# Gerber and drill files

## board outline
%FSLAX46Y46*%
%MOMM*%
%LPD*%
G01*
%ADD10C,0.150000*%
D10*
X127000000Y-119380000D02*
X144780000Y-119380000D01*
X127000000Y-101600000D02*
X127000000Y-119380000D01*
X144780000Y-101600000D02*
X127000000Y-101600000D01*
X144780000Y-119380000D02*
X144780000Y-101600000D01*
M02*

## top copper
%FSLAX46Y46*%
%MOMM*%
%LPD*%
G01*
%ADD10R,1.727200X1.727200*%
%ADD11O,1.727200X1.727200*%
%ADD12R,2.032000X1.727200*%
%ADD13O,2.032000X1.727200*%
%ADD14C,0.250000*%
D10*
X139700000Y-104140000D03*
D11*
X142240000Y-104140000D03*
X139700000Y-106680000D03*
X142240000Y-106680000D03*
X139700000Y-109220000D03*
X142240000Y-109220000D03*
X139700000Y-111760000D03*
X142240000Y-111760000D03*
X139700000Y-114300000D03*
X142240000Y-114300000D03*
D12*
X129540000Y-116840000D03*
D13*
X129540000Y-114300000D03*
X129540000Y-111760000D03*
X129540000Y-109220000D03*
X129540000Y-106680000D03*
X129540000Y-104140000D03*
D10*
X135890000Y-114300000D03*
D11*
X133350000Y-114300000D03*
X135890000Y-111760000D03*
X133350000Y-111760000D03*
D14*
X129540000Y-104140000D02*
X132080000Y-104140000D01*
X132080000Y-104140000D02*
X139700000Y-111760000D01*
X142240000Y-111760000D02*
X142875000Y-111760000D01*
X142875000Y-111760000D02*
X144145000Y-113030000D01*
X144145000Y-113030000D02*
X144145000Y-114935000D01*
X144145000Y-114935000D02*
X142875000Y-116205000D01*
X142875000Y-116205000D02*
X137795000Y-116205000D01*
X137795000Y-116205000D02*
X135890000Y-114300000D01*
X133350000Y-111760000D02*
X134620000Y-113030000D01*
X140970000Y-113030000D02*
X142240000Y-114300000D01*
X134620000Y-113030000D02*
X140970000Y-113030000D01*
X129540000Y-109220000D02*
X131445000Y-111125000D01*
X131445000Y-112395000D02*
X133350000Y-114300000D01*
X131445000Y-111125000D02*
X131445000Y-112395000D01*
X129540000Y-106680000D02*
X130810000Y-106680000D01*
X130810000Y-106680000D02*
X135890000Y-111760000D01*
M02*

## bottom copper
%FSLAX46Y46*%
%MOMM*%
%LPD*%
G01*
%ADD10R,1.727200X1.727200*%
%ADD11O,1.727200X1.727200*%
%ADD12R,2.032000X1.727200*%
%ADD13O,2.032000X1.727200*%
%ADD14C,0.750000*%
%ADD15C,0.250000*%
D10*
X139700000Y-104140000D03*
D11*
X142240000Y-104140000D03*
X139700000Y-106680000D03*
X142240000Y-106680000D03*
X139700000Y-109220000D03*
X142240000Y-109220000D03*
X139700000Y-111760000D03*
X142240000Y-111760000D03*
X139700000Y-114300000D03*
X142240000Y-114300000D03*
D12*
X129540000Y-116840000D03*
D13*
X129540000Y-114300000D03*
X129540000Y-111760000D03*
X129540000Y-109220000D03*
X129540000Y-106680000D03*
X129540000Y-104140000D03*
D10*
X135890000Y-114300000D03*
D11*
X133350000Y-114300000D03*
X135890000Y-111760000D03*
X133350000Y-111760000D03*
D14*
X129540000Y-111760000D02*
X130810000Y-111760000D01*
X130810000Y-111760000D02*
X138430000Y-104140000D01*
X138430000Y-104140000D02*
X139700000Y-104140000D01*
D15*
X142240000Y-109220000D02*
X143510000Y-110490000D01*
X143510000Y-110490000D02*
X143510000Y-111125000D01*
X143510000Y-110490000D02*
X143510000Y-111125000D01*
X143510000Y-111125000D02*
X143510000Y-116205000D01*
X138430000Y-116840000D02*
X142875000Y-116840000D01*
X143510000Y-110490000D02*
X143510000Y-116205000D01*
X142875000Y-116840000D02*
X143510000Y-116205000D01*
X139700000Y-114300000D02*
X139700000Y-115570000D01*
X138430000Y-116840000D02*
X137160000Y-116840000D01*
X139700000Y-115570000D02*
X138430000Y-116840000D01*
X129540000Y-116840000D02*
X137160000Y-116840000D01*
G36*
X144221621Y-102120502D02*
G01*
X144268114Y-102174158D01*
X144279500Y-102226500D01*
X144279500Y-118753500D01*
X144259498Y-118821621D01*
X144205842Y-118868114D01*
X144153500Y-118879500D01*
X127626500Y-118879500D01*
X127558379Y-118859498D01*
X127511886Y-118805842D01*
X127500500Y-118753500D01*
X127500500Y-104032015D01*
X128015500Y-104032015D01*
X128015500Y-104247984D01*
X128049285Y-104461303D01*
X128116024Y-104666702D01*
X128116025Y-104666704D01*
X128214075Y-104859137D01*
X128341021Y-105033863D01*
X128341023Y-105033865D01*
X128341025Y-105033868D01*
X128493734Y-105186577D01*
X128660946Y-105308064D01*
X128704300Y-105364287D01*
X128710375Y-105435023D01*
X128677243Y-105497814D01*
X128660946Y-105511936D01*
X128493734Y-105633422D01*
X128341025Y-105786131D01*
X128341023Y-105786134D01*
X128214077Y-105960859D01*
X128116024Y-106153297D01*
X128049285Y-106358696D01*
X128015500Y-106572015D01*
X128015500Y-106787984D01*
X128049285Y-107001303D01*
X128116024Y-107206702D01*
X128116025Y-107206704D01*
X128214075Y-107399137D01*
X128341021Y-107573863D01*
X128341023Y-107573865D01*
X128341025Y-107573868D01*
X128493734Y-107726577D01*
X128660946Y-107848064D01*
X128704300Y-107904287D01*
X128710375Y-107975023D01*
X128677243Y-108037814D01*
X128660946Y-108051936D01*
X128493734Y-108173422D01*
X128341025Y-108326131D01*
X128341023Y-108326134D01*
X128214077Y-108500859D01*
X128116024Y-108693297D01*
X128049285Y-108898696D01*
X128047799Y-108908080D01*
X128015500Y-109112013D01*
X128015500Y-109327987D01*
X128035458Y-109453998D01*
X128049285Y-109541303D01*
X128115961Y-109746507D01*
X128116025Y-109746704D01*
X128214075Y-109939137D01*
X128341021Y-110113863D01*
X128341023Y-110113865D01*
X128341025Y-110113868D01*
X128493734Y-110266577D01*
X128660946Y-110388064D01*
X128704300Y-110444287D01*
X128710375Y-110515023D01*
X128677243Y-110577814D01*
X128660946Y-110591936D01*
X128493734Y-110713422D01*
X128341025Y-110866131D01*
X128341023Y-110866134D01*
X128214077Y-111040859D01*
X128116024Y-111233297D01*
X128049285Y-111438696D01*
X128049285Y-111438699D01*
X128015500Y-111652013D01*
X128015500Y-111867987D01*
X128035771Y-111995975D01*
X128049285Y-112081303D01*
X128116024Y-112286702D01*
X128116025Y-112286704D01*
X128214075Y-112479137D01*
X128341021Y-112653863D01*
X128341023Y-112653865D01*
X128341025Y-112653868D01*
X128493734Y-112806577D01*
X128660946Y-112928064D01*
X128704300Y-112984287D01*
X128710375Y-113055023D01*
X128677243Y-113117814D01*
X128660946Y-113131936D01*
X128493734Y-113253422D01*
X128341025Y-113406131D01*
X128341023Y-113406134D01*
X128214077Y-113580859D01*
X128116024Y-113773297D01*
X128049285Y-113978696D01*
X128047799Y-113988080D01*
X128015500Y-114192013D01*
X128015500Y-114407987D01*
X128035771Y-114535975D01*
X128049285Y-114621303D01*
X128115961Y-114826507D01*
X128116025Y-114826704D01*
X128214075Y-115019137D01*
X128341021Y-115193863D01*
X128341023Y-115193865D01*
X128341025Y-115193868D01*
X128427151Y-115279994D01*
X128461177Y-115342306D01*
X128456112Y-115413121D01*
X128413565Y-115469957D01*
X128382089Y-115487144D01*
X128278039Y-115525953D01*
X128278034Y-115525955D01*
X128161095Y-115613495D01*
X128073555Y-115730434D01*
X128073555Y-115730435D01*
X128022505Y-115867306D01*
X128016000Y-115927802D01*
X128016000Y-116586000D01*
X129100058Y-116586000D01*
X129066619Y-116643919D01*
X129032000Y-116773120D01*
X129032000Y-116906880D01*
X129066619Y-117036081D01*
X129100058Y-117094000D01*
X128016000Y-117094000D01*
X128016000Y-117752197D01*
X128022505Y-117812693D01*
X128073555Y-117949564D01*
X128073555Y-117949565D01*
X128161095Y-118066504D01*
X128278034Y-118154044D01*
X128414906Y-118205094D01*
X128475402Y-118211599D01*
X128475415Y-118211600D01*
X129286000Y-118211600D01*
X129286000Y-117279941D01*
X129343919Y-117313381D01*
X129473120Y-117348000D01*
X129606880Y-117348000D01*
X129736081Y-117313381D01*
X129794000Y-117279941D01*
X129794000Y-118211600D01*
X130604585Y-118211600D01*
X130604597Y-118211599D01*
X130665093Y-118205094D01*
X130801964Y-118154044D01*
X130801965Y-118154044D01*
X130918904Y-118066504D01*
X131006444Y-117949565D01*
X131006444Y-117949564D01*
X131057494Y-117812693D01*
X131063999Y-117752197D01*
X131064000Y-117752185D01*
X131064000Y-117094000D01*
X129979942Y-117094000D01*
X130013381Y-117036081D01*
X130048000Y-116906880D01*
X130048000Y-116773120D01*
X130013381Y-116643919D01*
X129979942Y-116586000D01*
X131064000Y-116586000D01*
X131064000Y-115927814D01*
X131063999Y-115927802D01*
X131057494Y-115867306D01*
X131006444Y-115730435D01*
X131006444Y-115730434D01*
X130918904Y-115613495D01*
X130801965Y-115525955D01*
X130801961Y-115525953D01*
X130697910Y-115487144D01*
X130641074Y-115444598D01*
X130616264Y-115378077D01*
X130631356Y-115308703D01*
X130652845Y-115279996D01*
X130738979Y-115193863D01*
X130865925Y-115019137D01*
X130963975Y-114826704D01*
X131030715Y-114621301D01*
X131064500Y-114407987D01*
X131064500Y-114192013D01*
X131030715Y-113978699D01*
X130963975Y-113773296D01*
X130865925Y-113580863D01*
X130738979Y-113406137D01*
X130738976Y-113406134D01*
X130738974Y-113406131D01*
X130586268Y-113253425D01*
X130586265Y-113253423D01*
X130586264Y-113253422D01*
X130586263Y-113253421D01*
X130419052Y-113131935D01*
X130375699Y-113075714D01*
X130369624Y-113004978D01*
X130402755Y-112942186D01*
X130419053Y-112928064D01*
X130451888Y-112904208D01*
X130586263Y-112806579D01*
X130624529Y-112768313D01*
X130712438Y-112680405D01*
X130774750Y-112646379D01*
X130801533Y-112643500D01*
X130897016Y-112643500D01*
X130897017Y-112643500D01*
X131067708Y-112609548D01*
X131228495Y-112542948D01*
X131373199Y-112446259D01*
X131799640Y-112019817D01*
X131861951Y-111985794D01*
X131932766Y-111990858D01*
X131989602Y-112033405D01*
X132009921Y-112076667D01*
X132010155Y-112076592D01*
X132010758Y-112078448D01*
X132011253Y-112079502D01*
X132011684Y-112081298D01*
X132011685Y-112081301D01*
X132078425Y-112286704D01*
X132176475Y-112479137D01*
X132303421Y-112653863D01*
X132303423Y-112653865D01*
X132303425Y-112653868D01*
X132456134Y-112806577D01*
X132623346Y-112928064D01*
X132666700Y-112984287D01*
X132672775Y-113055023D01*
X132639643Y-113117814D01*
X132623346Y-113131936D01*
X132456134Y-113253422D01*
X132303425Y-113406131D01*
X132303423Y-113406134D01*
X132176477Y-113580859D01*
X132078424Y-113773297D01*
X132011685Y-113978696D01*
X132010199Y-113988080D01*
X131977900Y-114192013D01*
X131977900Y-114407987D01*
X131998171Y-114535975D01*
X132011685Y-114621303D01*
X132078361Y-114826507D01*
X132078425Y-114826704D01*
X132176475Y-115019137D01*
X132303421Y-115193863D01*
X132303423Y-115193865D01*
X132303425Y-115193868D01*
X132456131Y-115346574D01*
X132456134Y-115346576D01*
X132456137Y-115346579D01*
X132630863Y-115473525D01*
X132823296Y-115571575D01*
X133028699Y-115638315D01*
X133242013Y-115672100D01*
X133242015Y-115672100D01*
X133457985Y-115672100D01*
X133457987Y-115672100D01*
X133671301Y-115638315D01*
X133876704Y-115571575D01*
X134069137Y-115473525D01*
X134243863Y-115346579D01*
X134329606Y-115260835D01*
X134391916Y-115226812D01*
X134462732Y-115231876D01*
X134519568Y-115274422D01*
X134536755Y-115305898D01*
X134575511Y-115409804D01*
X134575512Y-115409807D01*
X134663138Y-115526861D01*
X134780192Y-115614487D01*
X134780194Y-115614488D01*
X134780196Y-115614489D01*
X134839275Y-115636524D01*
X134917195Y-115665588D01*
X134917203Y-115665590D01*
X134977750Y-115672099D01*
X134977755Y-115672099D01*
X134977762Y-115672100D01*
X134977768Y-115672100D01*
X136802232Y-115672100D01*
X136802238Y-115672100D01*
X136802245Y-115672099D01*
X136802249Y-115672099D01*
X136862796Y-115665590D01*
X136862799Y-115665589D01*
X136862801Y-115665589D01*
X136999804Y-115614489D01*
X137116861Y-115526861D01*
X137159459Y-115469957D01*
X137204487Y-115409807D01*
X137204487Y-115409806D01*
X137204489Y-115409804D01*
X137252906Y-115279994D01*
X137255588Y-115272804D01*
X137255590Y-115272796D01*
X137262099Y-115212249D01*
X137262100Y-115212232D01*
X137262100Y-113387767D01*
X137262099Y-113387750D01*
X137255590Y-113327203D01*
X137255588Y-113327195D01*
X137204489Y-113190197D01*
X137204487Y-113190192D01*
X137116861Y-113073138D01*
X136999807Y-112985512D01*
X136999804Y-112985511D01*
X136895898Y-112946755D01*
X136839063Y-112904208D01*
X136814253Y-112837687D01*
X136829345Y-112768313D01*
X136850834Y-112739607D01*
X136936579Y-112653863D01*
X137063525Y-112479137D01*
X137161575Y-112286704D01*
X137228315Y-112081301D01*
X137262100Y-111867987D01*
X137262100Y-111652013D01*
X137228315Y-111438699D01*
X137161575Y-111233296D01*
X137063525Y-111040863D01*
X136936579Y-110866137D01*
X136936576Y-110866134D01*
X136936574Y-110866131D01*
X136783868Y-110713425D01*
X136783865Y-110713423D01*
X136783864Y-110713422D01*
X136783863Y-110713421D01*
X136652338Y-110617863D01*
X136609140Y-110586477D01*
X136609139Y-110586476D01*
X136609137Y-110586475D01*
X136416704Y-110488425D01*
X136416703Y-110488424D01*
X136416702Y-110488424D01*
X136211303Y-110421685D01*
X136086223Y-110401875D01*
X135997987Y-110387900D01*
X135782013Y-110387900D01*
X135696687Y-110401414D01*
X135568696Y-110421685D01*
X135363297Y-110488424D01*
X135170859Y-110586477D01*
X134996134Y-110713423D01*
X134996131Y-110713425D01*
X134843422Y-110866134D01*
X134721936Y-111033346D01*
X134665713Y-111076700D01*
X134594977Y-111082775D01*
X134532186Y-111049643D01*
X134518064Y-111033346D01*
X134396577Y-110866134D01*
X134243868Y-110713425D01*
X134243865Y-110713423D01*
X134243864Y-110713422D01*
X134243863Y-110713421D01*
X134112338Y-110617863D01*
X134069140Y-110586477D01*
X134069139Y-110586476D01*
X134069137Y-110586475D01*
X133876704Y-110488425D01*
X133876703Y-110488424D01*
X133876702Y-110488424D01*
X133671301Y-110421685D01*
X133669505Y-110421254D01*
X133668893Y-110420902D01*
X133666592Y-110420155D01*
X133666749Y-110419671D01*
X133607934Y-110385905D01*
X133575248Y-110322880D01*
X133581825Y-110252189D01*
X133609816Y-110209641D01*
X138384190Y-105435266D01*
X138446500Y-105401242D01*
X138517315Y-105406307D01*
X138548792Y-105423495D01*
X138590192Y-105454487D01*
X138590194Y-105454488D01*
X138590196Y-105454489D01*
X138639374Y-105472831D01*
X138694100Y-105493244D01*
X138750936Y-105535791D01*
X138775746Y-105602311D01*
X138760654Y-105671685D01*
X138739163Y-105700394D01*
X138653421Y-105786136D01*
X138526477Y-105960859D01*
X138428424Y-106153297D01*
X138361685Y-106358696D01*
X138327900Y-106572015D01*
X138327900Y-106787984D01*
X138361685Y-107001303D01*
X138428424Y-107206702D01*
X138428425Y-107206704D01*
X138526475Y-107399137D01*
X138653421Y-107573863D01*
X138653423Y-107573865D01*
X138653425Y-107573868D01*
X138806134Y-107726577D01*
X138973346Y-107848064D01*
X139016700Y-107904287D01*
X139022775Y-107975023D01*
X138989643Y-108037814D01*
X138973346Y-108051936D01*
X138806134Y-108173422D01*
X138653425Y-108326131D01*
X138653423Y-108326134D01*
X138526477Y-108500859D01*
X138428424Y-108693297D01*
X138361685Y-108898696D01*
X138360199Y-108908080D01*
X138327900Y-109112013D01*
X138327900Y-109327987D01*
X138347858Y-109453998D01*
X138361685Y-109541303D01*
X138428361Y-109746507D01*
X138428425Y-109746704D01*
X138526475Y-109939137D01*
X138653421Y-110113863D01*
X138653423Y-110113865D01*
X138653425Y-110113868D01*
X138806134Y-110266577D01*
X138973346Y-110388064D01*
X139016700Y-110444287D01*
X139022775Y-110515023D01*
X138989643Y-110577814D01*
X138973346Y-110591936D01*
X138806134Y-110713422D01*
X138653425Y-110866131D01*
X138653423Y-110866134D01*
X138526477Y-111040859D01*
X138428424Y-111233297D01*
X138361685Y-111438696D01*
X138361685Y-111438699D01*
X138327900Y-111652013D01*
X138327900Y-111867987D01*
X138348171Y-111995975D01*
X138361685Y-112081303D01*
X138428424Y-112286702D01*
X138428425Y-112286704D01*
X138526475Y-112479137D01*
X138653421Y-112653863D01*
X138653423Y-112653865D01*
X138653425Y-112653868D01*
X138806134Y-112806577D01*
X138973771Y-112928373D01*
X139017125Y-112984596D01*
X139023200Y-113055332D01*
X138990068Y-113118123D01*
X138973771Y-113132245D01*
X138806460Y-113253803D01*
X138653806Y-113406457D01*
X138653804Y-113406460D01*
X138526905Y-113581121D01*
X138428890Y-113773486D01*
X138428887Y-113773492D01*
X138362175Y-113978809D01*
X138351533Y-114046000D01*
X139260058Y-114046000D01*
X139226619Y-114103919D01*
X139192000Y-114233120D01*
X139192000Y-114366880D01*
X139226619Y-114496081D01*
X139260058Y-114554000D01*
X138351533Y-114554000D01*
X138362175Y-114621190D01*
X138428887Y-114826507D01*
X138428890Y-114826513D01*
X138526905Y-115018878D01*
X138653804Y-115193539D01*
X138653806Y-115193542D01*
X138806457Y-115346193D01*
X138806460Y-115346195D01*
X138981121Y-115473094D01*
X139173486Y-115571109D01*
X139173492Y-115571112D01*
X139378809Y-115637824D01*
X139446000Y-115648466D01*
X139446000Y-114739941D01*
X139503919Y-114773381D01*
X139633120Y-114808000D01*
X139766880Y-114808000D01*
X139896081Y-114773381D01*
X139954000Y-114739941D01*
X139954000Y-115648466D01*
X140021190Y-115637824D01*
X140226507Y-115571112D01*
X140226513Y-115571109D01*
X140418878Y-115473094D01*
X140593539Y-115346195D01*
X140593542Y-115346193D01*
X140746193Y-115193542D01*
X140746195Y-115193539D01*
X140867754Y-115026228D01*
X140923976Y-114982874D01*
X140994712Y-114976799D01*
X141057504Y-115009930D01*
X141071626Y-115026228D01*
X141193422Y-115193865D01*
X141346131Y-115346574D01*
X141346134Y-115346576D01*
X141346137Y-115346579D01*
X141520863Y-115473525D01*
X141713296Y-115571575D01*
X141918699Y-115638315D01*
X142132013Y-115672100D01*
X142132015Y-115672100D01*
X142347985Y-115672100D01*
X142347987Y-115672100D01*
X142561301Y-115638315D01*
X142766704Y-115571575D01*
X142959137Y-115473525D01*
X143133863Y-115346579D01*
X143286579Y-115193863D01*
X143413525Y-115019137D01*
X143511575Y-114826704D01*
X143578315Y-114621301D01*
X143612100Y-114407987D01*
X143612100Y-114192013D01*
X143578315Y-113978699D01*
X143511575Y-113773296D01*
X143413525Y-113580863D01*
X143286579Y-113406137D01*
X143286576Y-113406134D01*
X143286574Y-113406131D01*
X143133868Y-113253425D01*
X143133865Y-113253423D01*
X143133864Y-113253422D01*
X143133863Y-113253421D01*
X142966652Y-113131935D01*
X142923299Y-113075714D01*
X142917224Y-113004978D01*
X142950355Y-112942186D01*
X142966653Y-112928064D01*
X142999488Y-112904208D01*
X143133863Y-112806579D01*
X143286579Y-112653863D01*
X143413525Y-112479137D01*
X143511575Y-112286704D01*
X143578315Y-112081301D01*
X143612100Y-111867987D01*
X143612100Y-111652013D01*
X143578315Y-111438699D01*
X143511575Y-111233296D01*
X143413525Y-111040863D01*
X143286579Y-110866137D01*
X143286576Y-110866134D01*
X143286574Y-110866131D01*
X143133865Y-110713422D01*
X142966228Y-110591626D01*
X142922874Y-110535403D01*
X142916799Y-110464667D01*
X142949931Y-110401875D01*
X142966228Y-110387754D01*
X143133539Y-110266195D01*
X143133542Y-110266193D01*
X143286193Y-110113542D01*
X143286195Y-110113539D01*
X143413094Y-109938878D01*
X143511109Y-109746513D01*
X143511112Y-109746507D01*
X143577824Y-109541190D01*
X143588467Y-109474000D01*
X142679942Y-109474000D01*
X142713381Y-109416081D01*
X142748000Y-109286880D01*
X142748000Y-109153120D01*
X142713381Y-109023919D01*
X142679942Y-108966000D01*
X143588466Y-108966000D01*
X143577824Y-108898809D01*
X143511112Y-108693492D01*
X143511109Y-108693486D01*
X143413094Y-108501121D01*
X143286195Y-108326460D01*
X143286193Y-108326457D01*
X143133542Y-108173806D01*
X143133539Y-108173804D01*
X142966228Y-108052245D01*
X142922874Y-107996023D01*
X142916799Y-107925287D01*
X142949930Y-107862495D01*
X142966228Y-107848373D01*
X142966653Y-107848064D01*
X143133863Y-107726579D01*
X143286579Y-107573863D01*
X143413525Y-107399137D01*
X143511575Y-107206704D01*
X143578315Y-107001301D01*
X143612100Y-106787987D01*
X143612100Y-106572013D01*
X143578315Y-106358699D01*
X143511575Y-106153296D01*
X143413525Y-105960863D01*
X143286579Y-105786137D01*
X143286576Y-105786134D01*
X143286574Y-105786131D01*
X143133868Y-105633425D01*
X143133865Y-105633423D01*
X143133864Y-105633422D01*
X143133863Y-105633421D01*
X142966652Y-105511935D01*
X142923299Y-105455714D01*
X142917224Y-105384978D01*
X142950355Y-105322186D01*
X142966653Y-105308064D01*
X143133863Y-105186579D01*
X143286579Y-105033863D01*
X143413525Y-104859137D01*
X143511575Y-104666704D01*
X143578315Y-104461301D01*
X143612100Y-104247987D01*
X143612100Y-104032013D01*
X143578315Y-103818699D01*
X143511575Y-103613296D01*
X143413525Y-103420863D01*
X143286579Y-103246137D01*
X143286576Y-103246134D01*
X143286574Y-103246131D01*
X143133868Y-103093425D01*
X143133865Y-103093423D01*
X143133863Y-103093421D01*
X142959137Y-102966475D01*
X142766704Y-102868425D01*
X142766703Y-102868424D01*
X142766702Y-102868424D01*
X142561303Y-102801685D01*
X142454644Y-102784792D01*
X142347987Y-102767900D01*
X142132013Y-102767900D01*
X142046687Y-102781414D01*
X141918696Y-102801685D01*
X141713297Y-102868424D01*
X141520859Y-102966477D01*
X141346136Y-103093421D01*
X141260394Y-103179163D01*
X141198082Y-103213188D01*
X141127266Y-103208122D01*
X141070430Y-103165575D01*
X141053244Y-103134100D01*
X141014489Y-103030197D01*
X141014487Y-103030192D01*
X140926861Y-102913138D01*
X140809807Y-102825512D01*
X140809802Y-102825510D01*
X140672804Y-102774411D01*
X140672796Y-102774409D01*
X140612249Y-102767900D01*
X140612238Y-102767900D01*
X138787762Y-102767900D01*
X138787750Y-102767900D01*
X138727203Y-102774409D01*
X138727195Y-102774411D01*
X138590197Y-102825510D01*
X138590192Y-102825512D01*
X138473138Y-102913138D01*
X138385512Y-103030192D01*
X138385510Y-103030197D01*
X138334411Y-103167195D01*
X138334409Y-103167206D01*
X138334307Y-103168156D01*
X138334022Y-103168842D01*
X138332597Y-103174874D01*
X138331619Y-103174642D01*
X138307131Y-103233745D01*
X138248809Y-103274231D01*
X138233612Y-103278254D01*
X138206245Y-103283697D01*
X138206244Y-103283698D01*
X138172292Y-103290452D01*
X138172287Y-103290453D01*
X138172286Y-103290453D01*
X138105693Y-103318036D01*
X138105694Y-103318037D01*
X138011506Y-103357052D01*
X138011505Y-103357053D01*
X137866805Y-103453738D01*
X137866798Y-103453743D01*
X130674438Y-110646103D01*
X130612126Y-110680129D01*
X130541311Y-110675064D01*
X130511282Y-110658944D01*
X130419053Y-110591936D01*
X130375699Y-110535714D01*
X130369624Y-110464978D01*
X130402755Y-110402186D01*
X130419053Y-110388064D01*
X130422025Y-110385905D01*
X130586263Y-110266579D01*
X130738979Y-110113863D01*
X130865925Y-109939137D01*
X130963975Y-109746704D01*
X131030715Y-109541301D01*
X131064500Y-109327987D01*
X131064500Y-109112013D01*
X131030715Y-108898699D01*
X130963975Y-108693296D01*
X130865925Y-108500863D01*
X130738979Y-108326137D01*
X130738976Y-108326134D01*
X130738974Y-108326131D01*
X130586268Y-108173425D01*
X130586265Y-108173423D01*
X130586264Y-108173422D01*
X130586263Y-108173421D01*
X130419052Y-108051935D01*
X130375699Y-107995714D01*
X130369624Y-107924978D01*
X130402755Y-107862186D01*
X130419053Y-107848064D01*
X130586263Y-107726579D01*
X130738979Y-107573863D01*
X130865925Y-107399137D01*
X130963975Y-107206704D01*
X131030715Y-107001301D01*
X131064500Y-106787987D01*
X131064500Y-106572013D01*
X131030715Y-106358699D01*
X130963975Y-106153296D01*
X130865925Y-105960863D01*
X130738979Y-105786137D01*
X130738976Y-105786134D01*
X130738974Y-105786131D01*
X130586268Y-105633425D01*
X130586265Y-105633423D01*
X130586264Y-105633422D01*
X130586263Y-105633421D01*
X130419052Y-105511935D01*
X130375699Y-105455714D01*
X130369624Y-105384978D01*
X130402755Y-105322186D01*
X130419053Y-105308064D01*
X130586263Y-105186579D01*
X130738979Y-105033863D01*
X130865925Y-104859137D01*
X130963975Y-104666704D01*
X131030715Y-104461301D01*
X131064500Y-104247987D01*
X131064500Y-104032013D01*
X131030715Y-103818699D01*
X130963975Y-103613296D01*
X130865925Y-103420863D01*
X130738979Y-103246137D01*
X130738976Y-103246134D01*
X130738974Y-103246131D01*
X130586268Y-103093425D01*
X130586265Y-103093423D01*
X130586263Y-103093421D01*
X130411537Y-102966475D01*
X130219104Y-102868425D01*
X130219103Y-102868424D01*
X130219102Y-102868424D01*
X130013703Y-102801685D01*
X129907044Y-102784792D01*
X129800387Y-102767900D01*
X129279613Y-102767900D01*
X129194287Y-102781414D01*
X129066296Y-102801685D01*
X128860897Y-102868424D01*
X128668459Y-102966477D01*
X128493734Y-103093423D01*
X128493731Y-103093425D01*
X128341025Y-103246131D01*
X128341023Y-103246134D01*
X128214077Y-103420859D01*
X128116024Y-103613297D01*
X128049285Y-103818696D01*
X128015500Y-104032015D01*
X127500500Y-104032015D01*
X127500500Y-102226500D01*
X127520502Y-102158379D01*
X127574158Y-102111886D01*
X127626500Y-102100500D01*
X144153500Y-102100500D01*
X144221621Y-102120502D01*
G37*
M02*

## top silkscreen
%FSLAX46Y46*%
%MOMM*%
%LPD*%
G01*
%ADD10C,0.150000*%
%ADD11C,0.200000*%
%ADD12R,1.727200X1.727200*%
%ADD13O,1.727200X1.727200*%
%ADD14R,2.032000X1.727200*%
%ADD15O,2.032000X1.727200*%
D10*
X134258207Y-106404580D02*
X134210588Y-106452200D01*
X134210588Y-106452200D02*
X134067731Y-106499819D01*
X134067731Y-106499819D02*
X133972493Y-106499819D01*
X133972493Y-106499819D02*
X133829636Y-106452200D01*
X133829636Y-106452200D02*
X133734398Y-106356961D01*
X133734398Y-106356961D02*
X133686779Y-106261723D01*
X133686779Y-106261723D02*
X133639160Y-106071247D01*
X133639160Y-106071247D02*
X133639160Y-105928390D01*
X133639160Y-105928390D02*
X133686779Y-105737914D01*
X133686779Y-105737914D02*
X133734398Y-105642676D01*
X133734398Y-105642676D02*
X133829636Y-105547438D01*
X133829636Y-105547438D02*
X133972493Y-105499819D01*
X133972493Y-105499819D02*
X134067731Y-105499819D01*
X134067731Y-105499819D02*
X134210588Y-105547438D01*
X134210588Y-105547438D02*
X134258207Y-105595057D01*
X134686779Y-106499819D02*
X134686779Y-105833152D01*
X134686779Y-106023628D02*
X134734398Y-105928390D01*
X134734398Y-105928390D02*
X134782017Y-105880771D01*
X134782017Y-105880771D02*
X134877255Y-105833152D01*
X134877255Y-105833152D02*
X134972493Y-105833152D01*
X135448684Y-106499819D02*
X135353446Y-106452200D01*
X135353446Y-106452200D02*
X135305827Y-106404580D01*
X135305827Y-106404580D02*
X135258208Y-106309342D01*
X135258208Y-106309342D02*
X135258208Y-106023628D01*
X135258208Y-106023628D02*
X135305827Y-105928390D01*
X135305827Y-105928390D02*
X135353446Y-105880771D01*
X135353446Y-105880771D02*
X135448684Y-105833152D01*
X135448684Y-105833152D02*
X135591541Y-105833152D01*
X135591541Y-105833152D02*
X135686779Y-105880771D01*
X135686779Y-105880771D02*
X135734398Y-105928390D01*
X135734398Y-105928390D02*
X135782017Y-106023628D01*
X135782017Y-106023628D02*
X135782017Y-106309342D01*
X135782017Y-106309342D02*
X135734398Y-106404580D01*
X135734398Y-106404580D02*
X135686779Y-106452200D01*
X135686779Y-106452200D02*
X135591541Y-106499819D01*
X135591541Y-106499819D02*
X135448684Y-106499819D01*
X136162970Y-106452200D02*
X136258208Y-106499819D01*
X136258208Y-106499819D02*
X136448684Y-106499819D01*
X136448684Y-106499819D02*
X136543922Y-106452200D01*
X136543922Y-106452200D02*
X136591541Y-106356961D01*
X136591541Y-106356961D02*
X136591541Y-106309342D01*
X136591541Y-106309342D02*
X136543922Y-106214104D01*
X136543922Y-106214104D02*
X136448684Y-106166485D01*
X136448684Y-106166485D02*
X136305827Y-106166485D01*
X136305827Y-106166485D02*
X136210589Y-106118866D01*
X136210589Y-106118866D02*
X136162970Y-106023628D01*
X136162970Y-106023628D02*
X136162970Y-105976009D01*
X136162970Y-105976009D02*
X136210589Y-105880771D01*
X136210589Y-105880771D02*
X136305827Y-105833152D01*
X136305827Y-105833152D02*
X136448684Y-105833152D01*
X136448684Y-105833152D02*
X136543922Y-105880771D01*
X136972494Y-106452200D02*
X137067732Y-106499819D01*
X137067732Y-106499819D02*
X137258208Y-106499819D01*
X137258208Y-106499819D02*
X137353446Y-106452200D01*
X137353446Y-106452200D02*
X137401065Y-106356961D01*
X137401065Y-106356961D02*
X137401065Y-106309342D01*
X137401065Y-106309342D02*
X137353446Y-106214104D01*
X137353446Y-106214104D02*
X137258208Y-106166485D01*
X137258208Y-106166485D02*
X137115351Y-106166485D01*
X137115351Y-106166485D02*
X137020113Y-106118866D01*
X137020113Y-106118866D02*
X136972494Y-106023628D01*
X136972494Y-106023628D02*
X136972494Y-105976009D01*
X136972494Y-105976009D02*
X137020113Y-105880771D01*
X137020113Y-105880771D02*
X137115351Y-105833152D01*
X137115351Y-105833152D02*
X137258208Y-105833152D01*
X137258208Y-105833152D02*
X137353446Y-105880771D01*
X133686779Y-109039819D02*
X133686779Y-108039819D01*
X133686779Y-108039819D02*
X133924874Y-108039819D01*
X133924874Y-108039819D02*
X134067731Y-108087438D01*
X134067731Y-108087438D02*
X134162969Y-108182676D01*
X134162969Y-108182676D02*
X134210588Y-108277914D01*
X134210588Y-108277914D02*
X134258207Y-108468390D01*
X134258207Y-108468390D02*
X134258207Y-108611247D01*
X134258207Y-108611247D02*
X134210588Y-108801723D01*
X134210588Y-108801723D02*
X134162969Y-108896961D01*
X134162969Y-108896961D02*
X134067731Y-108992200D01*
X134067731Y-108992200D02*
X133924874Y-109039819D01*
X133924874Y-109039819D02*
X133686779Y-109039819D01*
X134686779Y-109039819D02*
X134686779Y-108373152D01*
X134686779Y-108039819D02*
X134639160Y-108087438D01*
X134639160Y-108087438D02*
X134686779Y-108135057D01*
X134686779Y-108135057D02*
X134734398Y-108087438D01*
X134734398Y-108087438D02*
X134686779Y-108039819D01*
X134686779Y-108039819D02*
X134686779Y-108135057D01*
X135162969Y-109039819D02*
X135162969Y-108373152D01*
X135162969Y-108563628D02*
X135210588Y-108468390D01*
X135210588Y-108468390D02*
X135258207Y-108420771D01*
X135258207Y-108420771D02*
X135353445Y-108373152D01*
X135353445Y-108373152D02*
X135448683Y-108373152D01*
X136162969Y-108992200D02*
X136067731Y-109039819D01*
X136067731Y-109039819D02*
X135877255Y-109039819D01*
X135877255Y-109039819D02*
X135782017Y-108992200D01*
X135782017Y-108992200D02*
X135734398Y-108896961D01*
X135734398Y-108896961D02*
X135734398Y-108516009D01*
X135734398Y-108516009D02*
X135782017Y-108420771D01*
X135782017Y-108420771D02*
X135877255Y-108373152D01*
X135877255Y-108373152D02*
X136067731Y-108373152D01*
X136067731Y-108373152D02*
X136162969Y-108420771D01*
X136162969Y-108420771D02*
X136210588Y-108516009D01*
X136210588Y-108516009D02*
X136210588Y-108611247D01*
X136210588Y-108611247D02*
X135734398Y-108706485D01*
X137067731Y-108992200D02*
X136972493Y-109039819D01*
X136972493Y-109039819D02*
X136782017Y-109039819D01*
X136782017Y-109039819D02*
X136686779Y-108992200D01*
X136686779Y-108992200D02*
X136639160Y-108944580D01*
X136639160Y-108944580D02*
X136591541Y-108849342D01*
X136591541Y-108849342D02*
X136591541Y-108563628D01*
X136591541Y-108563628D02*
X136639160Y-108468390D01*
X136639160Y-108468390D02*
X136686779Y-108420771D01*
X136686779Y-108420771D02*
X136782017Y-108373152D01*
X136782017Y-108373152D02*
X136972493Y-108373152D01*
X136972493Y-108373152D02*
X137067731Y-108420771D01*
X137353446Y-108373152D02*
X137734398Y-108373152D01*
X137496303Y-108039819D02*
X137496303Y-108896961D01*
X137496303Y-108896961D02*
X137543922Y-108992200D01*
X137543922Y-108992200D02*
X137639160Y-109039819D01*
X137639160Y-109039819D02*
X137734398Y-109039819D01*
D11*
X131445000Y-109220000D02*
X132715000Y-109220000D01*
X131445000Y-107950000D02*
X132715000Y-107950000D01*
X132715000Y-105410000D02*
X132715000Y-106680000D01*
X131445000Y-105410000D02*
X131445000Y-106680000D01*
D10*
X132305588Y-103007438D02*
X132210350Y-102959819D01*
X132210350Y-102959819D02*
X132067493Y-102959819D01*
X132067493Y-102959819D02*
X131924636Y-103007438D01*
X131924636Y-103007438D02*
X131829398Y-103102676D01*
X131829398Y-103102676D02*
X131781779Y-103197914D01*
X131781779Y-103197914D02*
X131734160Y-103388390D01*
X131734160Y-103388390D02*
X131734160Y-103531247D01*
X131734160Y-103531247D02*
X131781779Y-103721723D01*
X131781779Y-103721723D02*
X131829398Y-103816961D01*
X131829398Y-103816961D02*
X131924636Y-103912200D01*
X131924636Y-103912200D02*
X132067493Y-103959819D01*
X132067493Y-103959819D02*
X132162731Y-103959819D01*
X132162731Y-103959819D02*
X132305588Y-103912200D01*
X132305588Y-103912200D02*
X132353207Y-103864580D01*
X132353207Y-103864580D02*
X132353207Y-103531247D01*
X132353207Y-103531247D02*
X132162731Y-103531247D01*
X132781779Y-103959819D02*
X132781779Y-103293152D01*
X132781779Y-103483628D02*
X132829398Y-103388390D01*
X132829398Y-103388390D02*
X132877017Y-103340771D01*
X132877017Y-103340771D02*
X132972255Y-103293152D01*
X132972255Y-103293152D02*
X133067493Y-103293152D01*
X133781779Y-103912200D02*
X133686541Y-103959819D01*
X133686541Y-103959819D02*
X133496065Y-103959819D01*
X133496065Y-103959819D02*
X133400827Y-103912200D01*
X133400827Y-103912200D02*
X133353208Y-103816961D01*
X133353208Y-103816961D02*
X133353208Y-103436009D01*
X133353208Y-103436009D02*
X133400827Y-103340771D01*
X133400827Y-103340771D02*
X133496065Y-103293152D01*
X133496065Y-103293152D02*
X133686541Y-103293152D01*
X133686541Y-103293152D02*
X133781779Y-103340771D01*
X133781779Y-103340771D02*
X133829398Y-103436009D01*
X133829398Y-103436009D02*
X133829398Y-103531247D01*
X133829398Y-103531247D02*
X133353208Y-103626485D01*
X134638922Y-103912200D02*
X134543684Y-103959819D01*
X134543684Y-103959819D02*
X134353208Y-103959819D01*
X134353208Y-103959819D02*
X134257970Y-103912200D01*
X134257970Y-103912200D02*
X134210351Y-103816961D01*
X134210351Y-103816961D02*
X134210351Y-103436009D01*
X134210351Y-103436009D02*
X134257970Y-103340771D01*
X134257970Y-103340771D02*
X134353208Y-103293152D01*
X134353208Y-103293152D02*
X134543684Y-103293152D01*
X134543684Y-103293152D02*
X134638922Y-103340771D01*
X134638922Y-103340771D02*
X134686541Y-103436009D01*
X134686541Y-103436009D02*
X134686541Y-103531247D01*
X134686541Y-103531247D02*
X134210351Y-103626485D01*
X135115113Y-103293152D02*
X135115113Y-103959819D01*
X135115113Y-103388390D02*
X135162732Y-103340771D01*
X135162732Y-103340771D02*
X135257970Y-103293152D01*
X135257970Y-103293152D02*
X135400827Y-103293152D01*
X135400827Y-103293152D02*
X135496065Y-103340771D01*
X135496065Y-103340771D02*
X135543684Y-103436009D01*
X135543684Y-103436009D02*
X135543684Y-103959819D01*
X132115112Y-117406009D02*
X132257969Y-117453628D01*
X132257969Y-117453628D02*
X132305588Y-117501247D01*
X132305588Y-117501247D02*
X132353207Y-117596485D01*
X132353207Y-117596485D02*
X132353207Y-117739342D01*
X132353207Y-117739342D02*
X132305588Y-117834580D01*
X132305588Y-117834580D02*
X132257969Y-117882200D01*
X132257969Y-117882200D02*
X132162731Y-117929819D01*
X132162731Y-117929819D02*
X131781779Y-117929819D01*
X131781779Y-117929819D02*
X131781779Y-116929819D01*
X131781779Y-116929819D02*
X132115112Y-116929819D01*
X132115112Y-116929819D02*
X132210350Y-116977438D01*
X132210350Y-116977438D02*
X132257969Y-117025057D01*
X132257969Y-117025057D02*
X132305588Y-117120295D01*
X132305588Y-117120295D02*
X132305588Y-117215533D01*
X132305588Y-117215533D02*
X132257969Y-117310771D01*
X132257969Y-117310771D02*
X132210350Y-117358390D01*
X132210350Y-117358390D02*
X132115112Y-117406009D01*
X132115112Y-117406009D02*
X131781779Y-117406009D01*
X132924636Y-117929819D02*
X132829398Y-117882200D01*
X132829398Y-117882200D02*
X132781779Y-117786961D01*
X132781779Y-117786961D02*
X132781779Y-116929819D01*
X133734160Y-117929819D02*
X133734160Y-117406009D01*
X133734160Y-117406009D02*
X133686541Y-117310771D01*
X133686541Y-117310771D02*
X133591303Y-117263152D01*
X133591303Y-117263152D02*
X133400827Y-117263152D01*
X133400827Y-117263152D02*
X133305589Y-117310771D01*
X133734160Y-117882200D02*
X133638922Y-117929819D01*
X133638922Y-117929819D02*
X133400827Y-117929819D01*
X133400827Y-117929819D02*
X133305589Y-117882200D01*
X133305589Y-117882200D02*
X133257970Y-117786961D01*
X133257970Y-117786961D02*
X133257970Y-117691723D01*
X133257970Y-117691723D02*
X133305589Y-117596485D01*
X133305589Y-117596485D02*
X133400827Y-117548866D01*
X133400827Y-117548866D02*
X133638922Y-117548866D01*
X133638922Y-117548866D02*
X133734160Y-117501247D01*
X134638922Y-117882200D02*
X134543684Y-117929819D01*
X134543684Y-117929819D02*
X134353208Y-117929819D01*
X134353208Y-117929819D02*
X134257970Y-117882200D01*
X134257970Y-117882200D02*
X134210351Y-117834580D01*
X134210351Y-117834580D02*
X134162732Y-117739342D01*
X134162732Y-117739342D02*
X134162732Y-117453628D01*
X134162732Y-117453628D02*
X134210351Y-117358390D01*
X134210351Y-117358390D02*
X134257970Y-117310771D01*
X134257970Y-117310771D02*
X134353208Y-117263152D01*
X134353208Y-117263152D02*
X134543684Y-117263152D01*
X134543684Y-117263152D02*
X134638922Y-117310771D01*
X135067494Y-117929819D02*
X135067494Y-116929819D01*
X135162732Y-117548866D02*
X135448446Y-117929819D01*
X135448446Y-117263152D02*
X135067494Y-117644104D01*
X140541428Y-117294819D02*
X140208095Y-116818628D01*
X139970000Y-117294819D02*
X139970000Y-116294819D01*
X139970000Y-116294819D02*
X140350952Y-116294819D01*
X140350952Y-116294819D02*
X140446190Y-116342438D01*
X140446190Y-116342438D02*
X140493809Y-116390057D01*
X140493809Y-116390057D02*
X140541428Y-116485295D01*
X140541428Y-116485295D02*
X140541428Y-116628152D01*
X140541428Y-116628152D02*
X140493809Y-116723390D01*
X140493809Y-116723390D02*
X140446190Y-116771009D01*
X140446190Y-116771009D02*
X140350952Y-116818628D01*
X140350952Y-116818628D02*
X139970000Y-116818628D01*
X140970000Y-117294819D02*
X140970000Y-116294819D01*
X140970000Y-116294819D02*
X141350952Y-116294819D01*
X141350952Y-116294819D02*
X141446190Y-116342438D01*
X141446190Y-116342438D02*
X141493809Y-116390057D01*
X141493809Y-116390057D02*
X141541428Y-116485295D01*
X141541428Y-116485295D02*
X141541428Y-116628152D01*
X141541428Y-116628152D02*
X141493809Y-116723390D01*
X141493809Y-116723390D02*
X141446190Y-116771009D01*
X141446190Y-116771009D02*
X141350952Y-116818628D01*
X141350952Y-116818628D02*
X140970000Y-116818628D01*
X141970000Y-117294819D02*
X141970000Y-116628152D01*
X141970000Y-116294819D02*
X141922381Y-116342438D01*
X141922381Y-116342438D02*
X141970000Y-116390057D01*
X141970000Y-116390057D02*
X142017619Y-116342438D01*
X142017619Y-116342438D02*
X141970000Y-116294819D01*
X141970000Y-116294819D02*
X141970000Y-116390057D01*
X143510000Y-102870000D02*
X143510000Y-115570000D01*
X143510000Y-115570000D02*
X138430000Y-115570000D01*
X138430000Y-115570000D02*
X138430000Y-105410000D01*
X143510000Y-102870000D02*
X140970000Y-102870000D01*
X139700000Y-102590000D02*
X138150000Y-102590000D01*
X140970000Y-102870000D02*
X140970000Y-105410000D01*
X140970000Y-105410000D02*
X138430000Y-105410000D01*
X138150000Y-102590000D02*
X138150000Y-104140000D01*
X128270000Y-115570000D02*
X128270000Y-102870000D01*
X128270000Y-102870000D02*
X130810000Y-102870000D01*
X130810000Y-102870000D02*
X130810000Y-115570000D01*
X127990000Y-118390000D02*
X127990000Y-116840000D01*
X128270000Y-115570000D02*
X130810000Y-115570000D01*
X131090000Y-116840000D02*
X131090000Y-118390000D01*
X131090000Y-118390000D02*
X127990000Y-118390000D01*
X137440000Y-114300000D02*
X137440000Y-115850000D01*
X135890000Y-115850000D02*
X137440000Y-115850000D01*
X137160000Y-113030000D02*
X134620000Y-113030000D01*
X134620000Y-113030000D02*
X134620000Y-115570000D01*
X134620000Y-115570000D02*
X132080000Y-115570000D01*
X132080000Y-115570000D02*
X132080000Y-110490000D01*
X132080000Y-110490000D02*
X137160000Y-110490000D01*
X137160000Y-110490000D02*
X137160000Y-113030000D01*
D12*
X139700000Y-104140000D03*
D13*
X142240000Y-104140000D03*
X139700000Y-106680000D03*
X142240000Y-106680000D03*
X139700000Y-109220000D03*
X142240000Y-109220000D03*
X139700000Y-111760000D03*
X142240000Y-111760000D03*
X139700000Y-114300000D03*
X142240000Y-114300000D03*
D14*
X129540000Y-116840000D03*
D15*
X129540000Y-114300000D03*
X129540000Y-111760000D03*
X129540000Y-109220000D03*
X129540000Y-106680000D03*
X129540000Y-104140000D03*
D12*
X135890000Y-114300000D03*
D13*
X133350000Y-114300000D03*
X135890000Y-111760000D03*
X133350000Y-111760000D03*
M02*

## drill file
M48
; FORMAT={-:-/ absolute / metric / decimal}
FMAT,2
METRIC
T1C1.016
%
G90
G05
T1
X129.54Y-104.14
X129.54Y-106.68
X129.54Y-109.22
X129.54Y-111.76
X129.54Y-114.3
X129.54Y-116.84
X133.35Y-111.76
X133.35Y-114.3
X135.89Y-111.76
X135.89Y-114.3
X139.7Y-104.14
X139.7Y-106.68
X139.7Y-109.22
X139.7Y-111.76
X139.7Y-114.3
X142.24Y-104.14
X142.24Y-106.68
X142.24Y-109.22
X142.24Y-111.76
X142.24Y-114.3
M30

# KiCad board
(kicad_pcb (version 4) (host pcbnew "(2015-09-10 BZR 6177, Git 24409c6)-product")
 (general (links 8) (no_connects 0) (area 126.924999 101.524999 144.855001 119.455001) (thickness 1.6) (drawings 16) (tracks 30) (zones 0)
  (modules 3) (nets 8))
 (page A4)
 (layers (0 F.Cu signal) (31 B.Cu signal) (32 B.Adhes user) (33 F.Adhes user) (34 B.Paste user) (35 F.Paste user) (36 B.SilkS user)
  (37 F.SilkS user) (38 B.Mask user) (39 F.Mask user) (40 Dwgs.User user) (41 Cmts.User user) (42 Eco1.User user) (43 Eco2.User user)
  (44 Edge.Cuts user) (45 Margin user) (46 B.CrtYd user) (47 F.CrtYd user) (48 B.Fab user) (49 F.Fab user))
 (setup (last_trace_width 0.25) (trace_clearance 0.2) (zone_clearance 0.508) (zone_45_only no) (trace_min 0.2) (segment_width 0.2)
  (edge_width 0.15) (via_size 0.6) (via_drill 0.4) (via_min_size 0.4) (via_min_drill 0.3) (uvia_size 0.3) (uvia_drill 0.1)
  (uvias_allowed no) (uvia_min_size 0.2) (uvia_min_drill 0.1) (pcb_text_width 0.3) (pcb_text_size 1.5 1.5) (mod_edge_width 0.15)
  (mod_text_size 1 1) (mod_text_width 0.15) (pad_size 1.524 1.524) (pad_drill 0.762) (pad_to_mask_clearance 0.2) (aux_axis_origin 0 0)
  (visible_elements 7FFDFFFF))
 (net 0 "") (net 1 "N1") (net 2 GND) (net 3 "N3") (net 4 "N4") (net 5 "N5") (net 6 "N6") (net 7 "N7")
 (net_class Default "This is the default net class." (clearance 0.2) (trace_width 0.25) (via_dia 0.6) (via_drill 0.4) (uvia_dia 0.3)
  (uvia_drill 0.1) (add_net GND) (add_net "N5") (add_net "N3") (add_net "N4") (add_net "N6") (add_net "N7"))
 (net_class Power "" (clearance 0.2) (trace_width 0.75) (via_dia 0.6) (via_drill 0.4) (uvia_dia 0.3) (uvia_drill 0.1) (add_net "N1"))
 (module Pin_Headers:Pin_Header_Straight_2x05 (layer F.Cu) (at 139.7 104.14)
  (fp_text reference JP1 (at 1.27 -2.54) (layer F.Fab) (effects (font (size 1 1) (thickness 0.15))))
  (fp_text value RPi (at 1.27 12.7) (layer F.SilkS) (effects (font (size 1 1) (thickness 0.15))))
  (fp_line (start 3.81 -1.27) (end 3.81 11.43) (layer F.SilkS) (width 0.15))
  (fp_line (start 3.81 11.43) (end -1.27 11.43) (layer F.SilkS) (width 0.15))
  (fp_line (start -1.27 11.43) (end -1.27 1.27) (layer F.SilkS) (width 0.15))
  (fp_line (start 3.81 -1.27) (end 1.27 -1.27) (layer F.SilkS) (width 0.15))
  (fp_line (start 0 -1.55) (end -1.55 -1.55) (layer F.SilkS) (width 0.15))
  (fp_line (start 1.27 -1.27) (end 1.27 1.27) (layer F.SilkS) (width 0.15))
  (fp_line (start 1.27 1.27) (end -1.27 1.27) (layer F.SilkS) (width 0.15))
  (fp_line (start -1.55 -1.55) (end -1.55 0) (layer F.SilkS) (width 0.15))
  (pad 1 thru_hole rect (at 0 0) (size 1.7272 1.7272) (drill 1.016) (layers *.Cu *.Mask F.SilkS) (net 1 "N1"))
  (pad 2 thru_hole oval (at 2.54 0) (size 1.7272 1.7272) (drill 1.016) (layers *.Cu *.Mask F.SilkS))
  (pad 3 thru_hole oval (at 0 2.54) (size 1.7272 1.7272) (drill 1.016) (layers *.Cu *.Mask F.SilkS))
  (pad 4 thru_hole oval (at 2.54 2.54) (size 1.7272 1.7272) (drill 1.016) (layers *.Cu *.Mask F.SilkS))
  (pad 5 thru_hole oval (at 0 5.08) (size 1.7272 1.7272) (drill 1.016) (layers *.Cu *.Mask F.SilkS))
  (pad 6 thru_hole oval (at 2.54 5.08) (size 1.7272 1.7272) (drill 1.016) (layers *.Cu *.Mask F.SilkS) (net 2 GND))
  (pad 7 thru_hole oval (at 0 7.62) (size 1.7272 1.7272) (drill 1.016) (layers *.Cu *.Mask F.SilkS) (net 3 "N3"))
  (pad 8 thru_hole oval (at 2.54 7.62) (size 1.7272 1.7272) (drill 1.016) (layers *.Cu *.Mask F.SilkS) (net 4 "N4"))
  (pad 9 thru_hole oval (at 0 10.16) (size 1.7272 1.7272) (drill 1.016) (layers *.Cu *.Mask F.SilkS) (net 2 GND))
  (pad 10 thru_hole oval (at 2.54 10.16) (size 1.7272 1.7272) (drill 1.016) (layers *.Cu *.Mask F.SilkS) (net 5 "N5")))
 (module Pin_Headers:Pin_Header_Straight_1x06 (layer F.Cu) (at 129.54 116.84 180)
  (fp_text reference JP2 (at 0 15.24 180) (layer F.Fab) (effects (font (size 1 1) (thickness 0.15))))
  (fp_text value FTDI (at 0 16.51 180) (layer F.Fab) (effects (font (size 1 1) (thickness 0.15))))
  (fp_line (start 1.27 1.27) (end 1.27 13.97) (layer F.SilkS) (width 0.15))
  (fp_line (start 1.27 13.97) (end -1.27 13.97) (layer F.SilkS) (width 0.15))
  (fp_line (start -1.27 13.97) (end -1.27 1.27) (layer F.SilkS) (width 0.15))
  (fp_line (start 1.55 -1.55) (end 1.55 0) (layer F.SilkS) (width 0.15))
  (fp_line (start 1.27 1.27) (end -1.27 1.27) (layer F.SilkS) (width 0.15))
  (fp_line (start -1.55 0) (end -1.55 -1.55) (layer F.SilkS) (width 0.15))
  (fp_line (start -1.55 -1.55) (end 1.55 -1.55) (layer F.SilkS) (width 0.15))
  (pad 1 thru_hole rect (at 0 0 180) (size 2.032 1.7272) (drill 1.016) (layers *.Cu *.Mask F.SilkS) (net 2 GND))
  (pad 2 thru_hole oval (at 0 2.54 180) (size 2.032 1.7272) (drill 1.016) (layers *.Cu *.Mask F.SilkS))
  (pad 3 thru_hole oval (at 0 5.08 180) (size 2.032 1.7272) (drill 1.016) (layers *.Cu *.Mask F.SilkS) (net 1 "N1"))
  (pad 4 thru_hole oval (at 0 7.62 180) (size 2.032 1.7272) (drill 1.016) (layers *.Cu *.Mask F.SilkS) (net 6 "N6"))
  (pad 5 thru_hole oval (at 0 10.16 180) (size 2.032 1.7272) (drill 1.016) (layers *.Cu *.Mask F.SilkS) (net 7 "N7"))
  (pad 6 thru_hole oval (at 0 12.7 180) (size 2.032 1.7272) (drill 1.016) (layers *.Cu *.Mask F.SilkS) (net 3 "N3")))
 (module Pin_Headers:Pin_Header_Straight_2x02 (layer F.Cu) (at 135.89 114.3 180)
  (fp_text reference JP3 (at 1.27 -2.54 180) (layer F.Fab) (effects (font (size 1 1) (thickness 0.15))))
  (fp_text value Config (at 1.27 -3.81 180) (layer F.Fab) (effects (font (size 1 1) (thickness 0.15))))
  (fp_line (start -1.55 0) (end -1.55 -1.55) (layer F.SilkS) (width 0.15))
  (fp_line (start 0 -1.55) (end -1.55 -1.55) (layer F.SilkS) (width 0.15))
  (fp_line (start -1.27 1.27) (end 1.27 1.27) (layer F.SilkS) (width 0.15))
  (fp_line (start 1.27 1.27) (end 1.27 -1.27) (layer F.SilkS) (width 0.15))
  (fp_line (start 1.27 -1.27) (end 3.81 -1.27) (layer F.SilkS) (width 0.15))
  (fp_line (start 3.81 -1.27) (end 3.81 3.81) (layer F.SilkS) (width 0.15))
  (fp_line (start 3.81 3.81) (end -1.27 3.81) (layer F.SilkS) (width 0.15))
  (fp_line (start -1.27 3.81) (end -1.27 1.27) (layer F.SilkS) (width 0.15))
  (pad 1 thru_hole rect (at 0 0 180) (size 1.7272 1.7272) (drill 1.016) (layers *.Cu *.Mask F.SilkS) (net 4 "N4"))
  (pad 2 thru_hole oval (at 2.54 0 180) (size 1.7272 1.7272) (drill 1.016) (layers *.Cu *.Mask F.SilkS) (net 6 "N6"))
  (pad 3 thru_hole oval (at 0 2.54 180) (size 1.7272 1.7272) (drill 1.016) (layers *.Cu *.Mask F.SilkS) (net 7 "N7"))
  (pad 4 thru_hole oval (at 2.54 2.54 180) (size 1.7272 1.7272) (drill 1.016) (layers *.Cu *.Mask F.SilkS) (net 5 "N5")))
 (gr_line (start 127 119.38) (end 144.78 119.38) (angle 90) (layer Edge.Cuts) (width 0.15))
 (gr_line (start 127 101.6) (end 127 119.38) (angle 90) (layer Edge.Cuts) (width 0.15))
 (gr_line (start 144.78 101.6) (end 127 101.6) (angle 90) (layer Edge.Cuts) (width 0.15))
 (gr_line (start 144.78 119.38) (end 144.78 101.6) (angle 90) (layer Edge.Cuts) (width 0.15))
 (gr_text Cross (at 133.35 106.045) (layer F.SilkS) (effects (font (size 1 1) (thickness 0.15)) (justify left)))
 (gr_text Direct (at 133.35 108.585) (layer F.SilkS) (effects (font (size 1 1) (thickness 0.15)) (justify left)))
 (gr_line (start 131.445 109.22) (end 132.715 109.22) (angle 90) (layer F.SilkS) (width 0.2))
 (gr_line (start 131.445 107.95) (end 132.715 107.95) (angle 90) (layer F.SilkS) (width 0.2))
 (gr_line (start 132.715 105.41) (end 132.715 106.68) (angle 90) (layer F.SilkS) (width 0.2))
 (gr_line (start 131.445 105.41) (end 131.445 106.68) (angle 90) (layer F.SilkS) (width 0.2))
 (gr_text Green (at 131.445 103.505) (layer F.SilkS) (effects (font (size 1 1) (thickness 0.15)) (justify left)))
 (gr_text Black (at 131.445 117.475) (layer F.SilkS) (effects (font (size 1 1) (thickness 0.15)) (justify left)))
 (segment (start 129.54 111.76) (end 130.81 111.76) (width 0.75) (layer B.Cu) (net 1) (status 10))
 (segment (start 130.81 111.76) (end 138.43 104.14) (width 0.75) (layer B.Cu) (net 1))
 (segment (start 138.43 104.14) (end 139.7 104.14) (width 0.75) (layer B.Cu) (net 1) (status 20))
 (segment (start 129.54 104.14) (end 132.08 104.14) (width 0.25) (layer F.Cu) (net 3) (status 10))
 (segment (start 132.08 104.14) (end 139.7 111.76) (width 0.25) (layer F.Cu) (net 3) (status 20))
 (segment (start 142.24 111.76) (end 142.875 111.76) (width 0.25) (layer F.Cu) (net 4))
 (segment (start 142.875 111.76) (end 144.145 113.03) (width 0.25) (layer F.Cu) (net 4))
 (segment (start 144.145 113.03) (end 144.145 114.935) (width 0.25) (layer F.Cu) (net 4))
 (segment (start 144.145 114.935) (end 142.875 116.205) (width 0.25) (layer F.Cu) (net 4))
 (segment (start 142.875 116.205) (end 137.795 116.205) (width 0.25) (layer F.Cu) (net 4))
 (segment (start 137.795 116.205) (end 135.89 114.3) (width 0.25) (layer F.Cu) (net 4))
 (segment (start 133.35 111.76) (end 134.62 113.03) (width 0.25) (layer F.Cu) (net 5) (status 10))
 (segment (start 140.97 113.03) (end 142.24 114.3) (width 0.25) (layer F.Cu) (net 5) (status 20))
 (segment (start 134.62 113.03) (end 140.97 113.03) (width 0.25) (layer F.Cu) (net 5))
 (segment (start 129.54 109.22) (end 131.445 111.125) (width 0.25) (layer F.Cu) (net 6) (status 10))
 (segment (start 131.445 112.395) (end 133.35 114.3) (width 0.25) (layer F.Cu) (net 6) (status 20))
 (segment (start 131.445 111.125) (end 131.445 112.395) (width 0.25) (layer F.Cu) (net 6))
 (segment (start 129.54 106.68) (end 130.81 106.68) (width 0.25) (layer F.Cu) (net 7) (status 10))
 (segment (start 130.81 106.68) (end 135.89 111.76) (width 0.25) (layer F.Cu) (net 7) (status 20))
 (segment (start 142.24 109.22) (end 143.51 110.49) (width 0.25) (layer B.Cu) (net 2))
 (segment (start 143.51 110.49) (end 143.51 111.125) (width 0.25) (layer B.Cu) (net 2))
 (segment (start 143.51 110.49) (end 143.51 111.125) (width 0.25) (layer B.Cu) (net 2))
 (segment (start 143.51 111.125) (end 143.51 116.205) (width 0.25) (layer B.Cu) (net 2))
 (segment (start 138.43 116.84) (end 142.875 116.84) (width 0.25) (layer B.Cu) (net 2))
 (segment (start 143.51 110.49) (end 143.51 116.205) (width 0.25) (layer B.Cu) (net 2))
 (segment (start 142.875 116.84) (end 143.51 116.205) (width 0.25) (layer B.Cu) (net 2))
 (segment (start 139.7 114.3) (end 139.7 115.57) (width 0.25) (layer B.Cu) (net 2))
 (segment (start 138.43 116.84) (end 137.16 116.84) (width 0.25) (layer B.Cu) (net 2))
 (segment (start 139.7 115.57) (end 138.43 116.84) (width 0.25) (layer B.Cu) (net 2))
 (segment (start 129.54 116.84) (end 137.16 116.84) (width 0.25) (layer B.Cu) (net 2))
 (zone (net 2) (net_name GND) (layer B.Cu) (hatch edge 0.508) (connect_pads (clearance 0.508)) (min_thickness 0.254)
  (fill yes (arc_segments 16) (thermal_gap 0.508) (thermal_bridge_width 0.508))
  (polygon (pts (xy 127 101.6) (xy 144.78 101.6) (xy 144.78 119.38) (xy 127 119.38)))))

